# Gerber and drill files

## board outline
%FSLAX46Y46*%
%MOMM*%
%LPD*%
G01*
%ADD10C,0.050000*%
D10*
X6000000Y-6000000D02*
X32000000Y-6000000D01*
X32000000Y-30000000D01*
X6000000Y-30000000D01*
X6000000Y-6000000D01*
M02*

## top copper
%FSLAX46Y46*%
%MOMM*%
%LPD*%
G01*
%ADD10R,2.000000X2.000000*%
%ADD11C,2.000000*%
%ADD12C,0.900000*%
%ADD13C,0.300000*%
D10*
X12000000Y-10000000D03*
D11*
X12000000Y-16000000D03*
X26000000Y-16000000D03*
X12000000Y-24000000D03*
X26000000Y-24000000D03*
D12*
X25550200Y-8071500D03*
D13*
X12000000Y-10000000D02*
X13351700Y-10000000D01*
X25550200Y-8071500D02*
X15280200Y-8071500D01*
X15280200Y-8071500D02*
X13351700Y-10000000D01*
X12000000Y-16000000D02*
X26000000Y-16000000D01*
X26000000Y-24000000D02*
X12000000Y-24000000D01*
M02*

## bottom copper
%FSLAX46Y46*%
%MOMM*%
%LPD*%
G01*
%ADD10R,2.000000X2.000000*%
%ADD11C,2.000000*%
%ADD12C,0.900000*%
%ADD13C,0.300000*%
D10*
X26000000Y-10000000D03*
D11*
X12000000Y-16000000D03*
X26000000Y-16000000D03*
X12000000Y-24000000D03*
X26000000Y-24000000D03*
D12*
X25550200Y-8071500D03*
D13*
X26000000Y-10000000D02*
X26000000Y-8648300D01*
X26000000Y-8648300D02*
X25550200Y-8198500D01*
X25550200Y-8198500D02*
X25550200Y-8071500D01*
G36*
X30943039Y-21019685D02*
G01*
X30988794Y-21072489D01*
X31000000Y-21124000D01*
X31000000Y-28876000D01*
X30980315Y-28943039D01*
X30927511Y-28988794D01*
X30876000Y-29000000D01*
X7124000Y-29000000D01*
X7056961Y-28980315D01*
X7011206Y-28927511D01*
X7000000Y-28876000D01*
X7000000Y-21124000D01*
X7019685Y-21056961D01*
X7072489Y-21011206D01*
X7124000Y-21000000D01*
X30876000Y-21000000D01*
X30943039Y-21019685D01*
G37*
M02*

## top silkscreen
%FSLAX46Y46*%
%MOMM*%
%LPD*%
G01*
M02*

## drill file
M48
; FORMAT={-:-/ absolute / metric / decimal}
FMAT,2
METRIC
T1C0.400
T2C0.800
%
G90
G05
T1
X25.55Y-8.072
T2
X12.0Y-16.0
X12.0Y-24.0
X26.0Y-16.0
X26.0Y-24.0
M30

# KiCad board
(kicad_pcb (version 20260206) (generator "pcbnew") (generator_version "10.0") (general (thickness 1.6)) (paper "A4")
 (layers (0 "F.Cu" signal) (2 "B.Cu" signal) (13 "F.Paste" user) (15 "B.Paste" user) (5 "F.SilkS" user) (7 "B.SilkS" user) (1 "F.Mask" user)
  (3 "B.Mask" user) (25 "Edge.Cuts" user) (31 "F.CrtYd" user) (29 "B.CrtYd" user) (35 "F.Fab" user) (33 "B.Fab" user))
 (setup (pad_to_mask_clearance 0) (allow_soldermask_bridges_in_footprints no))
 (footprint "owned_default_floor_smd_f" (layer "F.Cu") (at 12 10)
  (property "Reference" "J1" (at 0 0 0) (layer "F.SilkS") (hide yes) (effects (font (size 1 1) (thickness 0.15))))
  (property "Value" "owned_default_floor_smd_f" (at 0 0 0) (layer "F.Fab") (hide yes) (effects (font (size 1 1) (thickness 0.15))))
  (pad "1" smd rect (at 0 0) (size 2 2) (layers "F.Cu" "F.Paste" "F.Mask") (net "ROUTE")))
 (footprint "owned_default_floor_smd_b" (layer "B.Cu") (at 26 10)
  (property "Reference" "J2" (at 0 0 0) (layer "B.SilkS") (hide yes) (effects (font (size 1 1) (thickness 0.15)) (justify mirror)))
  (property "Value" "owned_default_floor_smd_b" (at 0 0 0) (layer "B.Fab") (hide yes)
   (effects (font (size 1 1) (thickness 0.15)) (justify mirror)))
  (pad "1" smd rect (at 0 0) (size 2 2) (layers "B.Cu" "B.Paste" "B.Mask") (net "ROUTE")))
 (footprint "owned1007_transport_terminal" (layer "F.Cu") (at 12 16)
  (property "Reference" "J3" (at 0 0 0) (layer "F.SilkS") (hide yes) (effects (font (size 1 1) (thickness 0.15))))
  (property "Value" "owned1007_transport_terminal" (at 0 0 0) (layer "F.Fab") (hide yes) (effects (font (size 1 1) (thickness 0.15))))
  (pad "1" thru_hole circle (at 0 0) (size 2 2) (drill 0.8) (layers "*.Cu" "*.Mask") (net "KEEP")))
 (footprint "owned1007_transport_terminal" (layer "F.Cu") (at 26 16)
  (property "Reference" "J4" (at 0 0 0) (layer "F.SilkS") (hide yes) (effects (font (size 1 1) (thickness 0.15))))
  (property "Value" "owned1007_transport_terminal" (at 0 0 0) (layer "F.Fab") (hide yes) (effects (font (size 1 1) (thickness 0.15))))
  (pad "1" thru_hole circle (at 0 0) (size 2 2) (drill 0.8) (layers "*.Cu" "*.Mask") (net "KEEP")))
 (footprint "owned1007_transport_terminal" (layer "F.Cu") (at 12 24)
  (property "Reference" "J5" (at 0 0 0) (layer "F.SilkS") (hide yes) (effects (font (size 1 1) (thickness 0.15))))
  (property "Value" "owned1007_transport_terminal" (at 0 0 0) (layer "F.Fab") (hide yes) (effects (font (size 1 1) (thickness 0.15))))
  (pad "1" thru_hole circle (at 0 0) (size 2 2) (drill 0.8) (layers "*.Cu" "*.Mask") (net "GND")))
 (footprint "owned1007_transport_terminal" (layer "F.Cu") (at 26 24)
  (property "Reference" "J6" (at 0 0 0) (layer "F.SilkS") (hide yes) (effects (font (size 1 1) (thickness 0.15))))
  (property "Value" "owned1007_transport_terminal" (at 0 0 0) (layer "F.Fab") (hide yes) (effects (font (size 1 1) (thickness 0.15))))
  (pad "1" thru_hole circle (at 0 0) (size 2 2) (drill 0.8) (layers "*.Cu" "*.Mask") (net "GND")))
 (gr_rect (start 6 6) (end 32 30) (stroke (width 0.05) (type default)) (fill none) (layer "Edge.Cuts"))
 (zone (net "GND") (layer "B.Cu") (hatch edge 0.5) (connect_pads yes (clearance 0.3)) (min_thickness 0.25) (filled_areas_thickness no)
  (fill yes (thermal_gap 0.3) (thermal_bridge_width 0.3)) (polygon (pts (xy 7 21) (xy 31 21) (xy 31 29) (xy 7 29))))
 (segment (start 12 10) (end 13.3517 10) (width 0.3) (layer "F.Cu") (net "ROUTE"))
 (segment (start 25.5502 8.0715) (end 15.2802 8.0715) (width 0.3) (layer "F.Cu") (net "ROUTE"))
 (segment (start 15.2802 8.0715) (end 13.3517 10) (width 0.3) (layer "F.Cu") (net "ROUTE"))
 (via (at 25.5502 8.0715) (size 0.9) (drill 0.4) (layers "F.Cu" "B.Cu") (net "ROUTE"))
 (segment (start 26 10) (end 26 8.6483) (width 0.3) (layer "B.Cu") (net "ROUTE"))
 (segment (start 26 8.6483) (end 25.5502 8.1985) (width 0.3) (layer "B.Cu") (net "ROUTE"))
 (segment (start 25.5502 8.1985) (end 25.5502 8.0715) (width 0.3) (layer "B.Cu") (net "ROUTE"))
 (segment (start 12 16) (end 26 16) (width 0.3) (layer "F.Cu") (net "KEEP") (locked yes))
 (segment (start 26 24) (end 12 24) (width 0.3) (layer "F.Cu") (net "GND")))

